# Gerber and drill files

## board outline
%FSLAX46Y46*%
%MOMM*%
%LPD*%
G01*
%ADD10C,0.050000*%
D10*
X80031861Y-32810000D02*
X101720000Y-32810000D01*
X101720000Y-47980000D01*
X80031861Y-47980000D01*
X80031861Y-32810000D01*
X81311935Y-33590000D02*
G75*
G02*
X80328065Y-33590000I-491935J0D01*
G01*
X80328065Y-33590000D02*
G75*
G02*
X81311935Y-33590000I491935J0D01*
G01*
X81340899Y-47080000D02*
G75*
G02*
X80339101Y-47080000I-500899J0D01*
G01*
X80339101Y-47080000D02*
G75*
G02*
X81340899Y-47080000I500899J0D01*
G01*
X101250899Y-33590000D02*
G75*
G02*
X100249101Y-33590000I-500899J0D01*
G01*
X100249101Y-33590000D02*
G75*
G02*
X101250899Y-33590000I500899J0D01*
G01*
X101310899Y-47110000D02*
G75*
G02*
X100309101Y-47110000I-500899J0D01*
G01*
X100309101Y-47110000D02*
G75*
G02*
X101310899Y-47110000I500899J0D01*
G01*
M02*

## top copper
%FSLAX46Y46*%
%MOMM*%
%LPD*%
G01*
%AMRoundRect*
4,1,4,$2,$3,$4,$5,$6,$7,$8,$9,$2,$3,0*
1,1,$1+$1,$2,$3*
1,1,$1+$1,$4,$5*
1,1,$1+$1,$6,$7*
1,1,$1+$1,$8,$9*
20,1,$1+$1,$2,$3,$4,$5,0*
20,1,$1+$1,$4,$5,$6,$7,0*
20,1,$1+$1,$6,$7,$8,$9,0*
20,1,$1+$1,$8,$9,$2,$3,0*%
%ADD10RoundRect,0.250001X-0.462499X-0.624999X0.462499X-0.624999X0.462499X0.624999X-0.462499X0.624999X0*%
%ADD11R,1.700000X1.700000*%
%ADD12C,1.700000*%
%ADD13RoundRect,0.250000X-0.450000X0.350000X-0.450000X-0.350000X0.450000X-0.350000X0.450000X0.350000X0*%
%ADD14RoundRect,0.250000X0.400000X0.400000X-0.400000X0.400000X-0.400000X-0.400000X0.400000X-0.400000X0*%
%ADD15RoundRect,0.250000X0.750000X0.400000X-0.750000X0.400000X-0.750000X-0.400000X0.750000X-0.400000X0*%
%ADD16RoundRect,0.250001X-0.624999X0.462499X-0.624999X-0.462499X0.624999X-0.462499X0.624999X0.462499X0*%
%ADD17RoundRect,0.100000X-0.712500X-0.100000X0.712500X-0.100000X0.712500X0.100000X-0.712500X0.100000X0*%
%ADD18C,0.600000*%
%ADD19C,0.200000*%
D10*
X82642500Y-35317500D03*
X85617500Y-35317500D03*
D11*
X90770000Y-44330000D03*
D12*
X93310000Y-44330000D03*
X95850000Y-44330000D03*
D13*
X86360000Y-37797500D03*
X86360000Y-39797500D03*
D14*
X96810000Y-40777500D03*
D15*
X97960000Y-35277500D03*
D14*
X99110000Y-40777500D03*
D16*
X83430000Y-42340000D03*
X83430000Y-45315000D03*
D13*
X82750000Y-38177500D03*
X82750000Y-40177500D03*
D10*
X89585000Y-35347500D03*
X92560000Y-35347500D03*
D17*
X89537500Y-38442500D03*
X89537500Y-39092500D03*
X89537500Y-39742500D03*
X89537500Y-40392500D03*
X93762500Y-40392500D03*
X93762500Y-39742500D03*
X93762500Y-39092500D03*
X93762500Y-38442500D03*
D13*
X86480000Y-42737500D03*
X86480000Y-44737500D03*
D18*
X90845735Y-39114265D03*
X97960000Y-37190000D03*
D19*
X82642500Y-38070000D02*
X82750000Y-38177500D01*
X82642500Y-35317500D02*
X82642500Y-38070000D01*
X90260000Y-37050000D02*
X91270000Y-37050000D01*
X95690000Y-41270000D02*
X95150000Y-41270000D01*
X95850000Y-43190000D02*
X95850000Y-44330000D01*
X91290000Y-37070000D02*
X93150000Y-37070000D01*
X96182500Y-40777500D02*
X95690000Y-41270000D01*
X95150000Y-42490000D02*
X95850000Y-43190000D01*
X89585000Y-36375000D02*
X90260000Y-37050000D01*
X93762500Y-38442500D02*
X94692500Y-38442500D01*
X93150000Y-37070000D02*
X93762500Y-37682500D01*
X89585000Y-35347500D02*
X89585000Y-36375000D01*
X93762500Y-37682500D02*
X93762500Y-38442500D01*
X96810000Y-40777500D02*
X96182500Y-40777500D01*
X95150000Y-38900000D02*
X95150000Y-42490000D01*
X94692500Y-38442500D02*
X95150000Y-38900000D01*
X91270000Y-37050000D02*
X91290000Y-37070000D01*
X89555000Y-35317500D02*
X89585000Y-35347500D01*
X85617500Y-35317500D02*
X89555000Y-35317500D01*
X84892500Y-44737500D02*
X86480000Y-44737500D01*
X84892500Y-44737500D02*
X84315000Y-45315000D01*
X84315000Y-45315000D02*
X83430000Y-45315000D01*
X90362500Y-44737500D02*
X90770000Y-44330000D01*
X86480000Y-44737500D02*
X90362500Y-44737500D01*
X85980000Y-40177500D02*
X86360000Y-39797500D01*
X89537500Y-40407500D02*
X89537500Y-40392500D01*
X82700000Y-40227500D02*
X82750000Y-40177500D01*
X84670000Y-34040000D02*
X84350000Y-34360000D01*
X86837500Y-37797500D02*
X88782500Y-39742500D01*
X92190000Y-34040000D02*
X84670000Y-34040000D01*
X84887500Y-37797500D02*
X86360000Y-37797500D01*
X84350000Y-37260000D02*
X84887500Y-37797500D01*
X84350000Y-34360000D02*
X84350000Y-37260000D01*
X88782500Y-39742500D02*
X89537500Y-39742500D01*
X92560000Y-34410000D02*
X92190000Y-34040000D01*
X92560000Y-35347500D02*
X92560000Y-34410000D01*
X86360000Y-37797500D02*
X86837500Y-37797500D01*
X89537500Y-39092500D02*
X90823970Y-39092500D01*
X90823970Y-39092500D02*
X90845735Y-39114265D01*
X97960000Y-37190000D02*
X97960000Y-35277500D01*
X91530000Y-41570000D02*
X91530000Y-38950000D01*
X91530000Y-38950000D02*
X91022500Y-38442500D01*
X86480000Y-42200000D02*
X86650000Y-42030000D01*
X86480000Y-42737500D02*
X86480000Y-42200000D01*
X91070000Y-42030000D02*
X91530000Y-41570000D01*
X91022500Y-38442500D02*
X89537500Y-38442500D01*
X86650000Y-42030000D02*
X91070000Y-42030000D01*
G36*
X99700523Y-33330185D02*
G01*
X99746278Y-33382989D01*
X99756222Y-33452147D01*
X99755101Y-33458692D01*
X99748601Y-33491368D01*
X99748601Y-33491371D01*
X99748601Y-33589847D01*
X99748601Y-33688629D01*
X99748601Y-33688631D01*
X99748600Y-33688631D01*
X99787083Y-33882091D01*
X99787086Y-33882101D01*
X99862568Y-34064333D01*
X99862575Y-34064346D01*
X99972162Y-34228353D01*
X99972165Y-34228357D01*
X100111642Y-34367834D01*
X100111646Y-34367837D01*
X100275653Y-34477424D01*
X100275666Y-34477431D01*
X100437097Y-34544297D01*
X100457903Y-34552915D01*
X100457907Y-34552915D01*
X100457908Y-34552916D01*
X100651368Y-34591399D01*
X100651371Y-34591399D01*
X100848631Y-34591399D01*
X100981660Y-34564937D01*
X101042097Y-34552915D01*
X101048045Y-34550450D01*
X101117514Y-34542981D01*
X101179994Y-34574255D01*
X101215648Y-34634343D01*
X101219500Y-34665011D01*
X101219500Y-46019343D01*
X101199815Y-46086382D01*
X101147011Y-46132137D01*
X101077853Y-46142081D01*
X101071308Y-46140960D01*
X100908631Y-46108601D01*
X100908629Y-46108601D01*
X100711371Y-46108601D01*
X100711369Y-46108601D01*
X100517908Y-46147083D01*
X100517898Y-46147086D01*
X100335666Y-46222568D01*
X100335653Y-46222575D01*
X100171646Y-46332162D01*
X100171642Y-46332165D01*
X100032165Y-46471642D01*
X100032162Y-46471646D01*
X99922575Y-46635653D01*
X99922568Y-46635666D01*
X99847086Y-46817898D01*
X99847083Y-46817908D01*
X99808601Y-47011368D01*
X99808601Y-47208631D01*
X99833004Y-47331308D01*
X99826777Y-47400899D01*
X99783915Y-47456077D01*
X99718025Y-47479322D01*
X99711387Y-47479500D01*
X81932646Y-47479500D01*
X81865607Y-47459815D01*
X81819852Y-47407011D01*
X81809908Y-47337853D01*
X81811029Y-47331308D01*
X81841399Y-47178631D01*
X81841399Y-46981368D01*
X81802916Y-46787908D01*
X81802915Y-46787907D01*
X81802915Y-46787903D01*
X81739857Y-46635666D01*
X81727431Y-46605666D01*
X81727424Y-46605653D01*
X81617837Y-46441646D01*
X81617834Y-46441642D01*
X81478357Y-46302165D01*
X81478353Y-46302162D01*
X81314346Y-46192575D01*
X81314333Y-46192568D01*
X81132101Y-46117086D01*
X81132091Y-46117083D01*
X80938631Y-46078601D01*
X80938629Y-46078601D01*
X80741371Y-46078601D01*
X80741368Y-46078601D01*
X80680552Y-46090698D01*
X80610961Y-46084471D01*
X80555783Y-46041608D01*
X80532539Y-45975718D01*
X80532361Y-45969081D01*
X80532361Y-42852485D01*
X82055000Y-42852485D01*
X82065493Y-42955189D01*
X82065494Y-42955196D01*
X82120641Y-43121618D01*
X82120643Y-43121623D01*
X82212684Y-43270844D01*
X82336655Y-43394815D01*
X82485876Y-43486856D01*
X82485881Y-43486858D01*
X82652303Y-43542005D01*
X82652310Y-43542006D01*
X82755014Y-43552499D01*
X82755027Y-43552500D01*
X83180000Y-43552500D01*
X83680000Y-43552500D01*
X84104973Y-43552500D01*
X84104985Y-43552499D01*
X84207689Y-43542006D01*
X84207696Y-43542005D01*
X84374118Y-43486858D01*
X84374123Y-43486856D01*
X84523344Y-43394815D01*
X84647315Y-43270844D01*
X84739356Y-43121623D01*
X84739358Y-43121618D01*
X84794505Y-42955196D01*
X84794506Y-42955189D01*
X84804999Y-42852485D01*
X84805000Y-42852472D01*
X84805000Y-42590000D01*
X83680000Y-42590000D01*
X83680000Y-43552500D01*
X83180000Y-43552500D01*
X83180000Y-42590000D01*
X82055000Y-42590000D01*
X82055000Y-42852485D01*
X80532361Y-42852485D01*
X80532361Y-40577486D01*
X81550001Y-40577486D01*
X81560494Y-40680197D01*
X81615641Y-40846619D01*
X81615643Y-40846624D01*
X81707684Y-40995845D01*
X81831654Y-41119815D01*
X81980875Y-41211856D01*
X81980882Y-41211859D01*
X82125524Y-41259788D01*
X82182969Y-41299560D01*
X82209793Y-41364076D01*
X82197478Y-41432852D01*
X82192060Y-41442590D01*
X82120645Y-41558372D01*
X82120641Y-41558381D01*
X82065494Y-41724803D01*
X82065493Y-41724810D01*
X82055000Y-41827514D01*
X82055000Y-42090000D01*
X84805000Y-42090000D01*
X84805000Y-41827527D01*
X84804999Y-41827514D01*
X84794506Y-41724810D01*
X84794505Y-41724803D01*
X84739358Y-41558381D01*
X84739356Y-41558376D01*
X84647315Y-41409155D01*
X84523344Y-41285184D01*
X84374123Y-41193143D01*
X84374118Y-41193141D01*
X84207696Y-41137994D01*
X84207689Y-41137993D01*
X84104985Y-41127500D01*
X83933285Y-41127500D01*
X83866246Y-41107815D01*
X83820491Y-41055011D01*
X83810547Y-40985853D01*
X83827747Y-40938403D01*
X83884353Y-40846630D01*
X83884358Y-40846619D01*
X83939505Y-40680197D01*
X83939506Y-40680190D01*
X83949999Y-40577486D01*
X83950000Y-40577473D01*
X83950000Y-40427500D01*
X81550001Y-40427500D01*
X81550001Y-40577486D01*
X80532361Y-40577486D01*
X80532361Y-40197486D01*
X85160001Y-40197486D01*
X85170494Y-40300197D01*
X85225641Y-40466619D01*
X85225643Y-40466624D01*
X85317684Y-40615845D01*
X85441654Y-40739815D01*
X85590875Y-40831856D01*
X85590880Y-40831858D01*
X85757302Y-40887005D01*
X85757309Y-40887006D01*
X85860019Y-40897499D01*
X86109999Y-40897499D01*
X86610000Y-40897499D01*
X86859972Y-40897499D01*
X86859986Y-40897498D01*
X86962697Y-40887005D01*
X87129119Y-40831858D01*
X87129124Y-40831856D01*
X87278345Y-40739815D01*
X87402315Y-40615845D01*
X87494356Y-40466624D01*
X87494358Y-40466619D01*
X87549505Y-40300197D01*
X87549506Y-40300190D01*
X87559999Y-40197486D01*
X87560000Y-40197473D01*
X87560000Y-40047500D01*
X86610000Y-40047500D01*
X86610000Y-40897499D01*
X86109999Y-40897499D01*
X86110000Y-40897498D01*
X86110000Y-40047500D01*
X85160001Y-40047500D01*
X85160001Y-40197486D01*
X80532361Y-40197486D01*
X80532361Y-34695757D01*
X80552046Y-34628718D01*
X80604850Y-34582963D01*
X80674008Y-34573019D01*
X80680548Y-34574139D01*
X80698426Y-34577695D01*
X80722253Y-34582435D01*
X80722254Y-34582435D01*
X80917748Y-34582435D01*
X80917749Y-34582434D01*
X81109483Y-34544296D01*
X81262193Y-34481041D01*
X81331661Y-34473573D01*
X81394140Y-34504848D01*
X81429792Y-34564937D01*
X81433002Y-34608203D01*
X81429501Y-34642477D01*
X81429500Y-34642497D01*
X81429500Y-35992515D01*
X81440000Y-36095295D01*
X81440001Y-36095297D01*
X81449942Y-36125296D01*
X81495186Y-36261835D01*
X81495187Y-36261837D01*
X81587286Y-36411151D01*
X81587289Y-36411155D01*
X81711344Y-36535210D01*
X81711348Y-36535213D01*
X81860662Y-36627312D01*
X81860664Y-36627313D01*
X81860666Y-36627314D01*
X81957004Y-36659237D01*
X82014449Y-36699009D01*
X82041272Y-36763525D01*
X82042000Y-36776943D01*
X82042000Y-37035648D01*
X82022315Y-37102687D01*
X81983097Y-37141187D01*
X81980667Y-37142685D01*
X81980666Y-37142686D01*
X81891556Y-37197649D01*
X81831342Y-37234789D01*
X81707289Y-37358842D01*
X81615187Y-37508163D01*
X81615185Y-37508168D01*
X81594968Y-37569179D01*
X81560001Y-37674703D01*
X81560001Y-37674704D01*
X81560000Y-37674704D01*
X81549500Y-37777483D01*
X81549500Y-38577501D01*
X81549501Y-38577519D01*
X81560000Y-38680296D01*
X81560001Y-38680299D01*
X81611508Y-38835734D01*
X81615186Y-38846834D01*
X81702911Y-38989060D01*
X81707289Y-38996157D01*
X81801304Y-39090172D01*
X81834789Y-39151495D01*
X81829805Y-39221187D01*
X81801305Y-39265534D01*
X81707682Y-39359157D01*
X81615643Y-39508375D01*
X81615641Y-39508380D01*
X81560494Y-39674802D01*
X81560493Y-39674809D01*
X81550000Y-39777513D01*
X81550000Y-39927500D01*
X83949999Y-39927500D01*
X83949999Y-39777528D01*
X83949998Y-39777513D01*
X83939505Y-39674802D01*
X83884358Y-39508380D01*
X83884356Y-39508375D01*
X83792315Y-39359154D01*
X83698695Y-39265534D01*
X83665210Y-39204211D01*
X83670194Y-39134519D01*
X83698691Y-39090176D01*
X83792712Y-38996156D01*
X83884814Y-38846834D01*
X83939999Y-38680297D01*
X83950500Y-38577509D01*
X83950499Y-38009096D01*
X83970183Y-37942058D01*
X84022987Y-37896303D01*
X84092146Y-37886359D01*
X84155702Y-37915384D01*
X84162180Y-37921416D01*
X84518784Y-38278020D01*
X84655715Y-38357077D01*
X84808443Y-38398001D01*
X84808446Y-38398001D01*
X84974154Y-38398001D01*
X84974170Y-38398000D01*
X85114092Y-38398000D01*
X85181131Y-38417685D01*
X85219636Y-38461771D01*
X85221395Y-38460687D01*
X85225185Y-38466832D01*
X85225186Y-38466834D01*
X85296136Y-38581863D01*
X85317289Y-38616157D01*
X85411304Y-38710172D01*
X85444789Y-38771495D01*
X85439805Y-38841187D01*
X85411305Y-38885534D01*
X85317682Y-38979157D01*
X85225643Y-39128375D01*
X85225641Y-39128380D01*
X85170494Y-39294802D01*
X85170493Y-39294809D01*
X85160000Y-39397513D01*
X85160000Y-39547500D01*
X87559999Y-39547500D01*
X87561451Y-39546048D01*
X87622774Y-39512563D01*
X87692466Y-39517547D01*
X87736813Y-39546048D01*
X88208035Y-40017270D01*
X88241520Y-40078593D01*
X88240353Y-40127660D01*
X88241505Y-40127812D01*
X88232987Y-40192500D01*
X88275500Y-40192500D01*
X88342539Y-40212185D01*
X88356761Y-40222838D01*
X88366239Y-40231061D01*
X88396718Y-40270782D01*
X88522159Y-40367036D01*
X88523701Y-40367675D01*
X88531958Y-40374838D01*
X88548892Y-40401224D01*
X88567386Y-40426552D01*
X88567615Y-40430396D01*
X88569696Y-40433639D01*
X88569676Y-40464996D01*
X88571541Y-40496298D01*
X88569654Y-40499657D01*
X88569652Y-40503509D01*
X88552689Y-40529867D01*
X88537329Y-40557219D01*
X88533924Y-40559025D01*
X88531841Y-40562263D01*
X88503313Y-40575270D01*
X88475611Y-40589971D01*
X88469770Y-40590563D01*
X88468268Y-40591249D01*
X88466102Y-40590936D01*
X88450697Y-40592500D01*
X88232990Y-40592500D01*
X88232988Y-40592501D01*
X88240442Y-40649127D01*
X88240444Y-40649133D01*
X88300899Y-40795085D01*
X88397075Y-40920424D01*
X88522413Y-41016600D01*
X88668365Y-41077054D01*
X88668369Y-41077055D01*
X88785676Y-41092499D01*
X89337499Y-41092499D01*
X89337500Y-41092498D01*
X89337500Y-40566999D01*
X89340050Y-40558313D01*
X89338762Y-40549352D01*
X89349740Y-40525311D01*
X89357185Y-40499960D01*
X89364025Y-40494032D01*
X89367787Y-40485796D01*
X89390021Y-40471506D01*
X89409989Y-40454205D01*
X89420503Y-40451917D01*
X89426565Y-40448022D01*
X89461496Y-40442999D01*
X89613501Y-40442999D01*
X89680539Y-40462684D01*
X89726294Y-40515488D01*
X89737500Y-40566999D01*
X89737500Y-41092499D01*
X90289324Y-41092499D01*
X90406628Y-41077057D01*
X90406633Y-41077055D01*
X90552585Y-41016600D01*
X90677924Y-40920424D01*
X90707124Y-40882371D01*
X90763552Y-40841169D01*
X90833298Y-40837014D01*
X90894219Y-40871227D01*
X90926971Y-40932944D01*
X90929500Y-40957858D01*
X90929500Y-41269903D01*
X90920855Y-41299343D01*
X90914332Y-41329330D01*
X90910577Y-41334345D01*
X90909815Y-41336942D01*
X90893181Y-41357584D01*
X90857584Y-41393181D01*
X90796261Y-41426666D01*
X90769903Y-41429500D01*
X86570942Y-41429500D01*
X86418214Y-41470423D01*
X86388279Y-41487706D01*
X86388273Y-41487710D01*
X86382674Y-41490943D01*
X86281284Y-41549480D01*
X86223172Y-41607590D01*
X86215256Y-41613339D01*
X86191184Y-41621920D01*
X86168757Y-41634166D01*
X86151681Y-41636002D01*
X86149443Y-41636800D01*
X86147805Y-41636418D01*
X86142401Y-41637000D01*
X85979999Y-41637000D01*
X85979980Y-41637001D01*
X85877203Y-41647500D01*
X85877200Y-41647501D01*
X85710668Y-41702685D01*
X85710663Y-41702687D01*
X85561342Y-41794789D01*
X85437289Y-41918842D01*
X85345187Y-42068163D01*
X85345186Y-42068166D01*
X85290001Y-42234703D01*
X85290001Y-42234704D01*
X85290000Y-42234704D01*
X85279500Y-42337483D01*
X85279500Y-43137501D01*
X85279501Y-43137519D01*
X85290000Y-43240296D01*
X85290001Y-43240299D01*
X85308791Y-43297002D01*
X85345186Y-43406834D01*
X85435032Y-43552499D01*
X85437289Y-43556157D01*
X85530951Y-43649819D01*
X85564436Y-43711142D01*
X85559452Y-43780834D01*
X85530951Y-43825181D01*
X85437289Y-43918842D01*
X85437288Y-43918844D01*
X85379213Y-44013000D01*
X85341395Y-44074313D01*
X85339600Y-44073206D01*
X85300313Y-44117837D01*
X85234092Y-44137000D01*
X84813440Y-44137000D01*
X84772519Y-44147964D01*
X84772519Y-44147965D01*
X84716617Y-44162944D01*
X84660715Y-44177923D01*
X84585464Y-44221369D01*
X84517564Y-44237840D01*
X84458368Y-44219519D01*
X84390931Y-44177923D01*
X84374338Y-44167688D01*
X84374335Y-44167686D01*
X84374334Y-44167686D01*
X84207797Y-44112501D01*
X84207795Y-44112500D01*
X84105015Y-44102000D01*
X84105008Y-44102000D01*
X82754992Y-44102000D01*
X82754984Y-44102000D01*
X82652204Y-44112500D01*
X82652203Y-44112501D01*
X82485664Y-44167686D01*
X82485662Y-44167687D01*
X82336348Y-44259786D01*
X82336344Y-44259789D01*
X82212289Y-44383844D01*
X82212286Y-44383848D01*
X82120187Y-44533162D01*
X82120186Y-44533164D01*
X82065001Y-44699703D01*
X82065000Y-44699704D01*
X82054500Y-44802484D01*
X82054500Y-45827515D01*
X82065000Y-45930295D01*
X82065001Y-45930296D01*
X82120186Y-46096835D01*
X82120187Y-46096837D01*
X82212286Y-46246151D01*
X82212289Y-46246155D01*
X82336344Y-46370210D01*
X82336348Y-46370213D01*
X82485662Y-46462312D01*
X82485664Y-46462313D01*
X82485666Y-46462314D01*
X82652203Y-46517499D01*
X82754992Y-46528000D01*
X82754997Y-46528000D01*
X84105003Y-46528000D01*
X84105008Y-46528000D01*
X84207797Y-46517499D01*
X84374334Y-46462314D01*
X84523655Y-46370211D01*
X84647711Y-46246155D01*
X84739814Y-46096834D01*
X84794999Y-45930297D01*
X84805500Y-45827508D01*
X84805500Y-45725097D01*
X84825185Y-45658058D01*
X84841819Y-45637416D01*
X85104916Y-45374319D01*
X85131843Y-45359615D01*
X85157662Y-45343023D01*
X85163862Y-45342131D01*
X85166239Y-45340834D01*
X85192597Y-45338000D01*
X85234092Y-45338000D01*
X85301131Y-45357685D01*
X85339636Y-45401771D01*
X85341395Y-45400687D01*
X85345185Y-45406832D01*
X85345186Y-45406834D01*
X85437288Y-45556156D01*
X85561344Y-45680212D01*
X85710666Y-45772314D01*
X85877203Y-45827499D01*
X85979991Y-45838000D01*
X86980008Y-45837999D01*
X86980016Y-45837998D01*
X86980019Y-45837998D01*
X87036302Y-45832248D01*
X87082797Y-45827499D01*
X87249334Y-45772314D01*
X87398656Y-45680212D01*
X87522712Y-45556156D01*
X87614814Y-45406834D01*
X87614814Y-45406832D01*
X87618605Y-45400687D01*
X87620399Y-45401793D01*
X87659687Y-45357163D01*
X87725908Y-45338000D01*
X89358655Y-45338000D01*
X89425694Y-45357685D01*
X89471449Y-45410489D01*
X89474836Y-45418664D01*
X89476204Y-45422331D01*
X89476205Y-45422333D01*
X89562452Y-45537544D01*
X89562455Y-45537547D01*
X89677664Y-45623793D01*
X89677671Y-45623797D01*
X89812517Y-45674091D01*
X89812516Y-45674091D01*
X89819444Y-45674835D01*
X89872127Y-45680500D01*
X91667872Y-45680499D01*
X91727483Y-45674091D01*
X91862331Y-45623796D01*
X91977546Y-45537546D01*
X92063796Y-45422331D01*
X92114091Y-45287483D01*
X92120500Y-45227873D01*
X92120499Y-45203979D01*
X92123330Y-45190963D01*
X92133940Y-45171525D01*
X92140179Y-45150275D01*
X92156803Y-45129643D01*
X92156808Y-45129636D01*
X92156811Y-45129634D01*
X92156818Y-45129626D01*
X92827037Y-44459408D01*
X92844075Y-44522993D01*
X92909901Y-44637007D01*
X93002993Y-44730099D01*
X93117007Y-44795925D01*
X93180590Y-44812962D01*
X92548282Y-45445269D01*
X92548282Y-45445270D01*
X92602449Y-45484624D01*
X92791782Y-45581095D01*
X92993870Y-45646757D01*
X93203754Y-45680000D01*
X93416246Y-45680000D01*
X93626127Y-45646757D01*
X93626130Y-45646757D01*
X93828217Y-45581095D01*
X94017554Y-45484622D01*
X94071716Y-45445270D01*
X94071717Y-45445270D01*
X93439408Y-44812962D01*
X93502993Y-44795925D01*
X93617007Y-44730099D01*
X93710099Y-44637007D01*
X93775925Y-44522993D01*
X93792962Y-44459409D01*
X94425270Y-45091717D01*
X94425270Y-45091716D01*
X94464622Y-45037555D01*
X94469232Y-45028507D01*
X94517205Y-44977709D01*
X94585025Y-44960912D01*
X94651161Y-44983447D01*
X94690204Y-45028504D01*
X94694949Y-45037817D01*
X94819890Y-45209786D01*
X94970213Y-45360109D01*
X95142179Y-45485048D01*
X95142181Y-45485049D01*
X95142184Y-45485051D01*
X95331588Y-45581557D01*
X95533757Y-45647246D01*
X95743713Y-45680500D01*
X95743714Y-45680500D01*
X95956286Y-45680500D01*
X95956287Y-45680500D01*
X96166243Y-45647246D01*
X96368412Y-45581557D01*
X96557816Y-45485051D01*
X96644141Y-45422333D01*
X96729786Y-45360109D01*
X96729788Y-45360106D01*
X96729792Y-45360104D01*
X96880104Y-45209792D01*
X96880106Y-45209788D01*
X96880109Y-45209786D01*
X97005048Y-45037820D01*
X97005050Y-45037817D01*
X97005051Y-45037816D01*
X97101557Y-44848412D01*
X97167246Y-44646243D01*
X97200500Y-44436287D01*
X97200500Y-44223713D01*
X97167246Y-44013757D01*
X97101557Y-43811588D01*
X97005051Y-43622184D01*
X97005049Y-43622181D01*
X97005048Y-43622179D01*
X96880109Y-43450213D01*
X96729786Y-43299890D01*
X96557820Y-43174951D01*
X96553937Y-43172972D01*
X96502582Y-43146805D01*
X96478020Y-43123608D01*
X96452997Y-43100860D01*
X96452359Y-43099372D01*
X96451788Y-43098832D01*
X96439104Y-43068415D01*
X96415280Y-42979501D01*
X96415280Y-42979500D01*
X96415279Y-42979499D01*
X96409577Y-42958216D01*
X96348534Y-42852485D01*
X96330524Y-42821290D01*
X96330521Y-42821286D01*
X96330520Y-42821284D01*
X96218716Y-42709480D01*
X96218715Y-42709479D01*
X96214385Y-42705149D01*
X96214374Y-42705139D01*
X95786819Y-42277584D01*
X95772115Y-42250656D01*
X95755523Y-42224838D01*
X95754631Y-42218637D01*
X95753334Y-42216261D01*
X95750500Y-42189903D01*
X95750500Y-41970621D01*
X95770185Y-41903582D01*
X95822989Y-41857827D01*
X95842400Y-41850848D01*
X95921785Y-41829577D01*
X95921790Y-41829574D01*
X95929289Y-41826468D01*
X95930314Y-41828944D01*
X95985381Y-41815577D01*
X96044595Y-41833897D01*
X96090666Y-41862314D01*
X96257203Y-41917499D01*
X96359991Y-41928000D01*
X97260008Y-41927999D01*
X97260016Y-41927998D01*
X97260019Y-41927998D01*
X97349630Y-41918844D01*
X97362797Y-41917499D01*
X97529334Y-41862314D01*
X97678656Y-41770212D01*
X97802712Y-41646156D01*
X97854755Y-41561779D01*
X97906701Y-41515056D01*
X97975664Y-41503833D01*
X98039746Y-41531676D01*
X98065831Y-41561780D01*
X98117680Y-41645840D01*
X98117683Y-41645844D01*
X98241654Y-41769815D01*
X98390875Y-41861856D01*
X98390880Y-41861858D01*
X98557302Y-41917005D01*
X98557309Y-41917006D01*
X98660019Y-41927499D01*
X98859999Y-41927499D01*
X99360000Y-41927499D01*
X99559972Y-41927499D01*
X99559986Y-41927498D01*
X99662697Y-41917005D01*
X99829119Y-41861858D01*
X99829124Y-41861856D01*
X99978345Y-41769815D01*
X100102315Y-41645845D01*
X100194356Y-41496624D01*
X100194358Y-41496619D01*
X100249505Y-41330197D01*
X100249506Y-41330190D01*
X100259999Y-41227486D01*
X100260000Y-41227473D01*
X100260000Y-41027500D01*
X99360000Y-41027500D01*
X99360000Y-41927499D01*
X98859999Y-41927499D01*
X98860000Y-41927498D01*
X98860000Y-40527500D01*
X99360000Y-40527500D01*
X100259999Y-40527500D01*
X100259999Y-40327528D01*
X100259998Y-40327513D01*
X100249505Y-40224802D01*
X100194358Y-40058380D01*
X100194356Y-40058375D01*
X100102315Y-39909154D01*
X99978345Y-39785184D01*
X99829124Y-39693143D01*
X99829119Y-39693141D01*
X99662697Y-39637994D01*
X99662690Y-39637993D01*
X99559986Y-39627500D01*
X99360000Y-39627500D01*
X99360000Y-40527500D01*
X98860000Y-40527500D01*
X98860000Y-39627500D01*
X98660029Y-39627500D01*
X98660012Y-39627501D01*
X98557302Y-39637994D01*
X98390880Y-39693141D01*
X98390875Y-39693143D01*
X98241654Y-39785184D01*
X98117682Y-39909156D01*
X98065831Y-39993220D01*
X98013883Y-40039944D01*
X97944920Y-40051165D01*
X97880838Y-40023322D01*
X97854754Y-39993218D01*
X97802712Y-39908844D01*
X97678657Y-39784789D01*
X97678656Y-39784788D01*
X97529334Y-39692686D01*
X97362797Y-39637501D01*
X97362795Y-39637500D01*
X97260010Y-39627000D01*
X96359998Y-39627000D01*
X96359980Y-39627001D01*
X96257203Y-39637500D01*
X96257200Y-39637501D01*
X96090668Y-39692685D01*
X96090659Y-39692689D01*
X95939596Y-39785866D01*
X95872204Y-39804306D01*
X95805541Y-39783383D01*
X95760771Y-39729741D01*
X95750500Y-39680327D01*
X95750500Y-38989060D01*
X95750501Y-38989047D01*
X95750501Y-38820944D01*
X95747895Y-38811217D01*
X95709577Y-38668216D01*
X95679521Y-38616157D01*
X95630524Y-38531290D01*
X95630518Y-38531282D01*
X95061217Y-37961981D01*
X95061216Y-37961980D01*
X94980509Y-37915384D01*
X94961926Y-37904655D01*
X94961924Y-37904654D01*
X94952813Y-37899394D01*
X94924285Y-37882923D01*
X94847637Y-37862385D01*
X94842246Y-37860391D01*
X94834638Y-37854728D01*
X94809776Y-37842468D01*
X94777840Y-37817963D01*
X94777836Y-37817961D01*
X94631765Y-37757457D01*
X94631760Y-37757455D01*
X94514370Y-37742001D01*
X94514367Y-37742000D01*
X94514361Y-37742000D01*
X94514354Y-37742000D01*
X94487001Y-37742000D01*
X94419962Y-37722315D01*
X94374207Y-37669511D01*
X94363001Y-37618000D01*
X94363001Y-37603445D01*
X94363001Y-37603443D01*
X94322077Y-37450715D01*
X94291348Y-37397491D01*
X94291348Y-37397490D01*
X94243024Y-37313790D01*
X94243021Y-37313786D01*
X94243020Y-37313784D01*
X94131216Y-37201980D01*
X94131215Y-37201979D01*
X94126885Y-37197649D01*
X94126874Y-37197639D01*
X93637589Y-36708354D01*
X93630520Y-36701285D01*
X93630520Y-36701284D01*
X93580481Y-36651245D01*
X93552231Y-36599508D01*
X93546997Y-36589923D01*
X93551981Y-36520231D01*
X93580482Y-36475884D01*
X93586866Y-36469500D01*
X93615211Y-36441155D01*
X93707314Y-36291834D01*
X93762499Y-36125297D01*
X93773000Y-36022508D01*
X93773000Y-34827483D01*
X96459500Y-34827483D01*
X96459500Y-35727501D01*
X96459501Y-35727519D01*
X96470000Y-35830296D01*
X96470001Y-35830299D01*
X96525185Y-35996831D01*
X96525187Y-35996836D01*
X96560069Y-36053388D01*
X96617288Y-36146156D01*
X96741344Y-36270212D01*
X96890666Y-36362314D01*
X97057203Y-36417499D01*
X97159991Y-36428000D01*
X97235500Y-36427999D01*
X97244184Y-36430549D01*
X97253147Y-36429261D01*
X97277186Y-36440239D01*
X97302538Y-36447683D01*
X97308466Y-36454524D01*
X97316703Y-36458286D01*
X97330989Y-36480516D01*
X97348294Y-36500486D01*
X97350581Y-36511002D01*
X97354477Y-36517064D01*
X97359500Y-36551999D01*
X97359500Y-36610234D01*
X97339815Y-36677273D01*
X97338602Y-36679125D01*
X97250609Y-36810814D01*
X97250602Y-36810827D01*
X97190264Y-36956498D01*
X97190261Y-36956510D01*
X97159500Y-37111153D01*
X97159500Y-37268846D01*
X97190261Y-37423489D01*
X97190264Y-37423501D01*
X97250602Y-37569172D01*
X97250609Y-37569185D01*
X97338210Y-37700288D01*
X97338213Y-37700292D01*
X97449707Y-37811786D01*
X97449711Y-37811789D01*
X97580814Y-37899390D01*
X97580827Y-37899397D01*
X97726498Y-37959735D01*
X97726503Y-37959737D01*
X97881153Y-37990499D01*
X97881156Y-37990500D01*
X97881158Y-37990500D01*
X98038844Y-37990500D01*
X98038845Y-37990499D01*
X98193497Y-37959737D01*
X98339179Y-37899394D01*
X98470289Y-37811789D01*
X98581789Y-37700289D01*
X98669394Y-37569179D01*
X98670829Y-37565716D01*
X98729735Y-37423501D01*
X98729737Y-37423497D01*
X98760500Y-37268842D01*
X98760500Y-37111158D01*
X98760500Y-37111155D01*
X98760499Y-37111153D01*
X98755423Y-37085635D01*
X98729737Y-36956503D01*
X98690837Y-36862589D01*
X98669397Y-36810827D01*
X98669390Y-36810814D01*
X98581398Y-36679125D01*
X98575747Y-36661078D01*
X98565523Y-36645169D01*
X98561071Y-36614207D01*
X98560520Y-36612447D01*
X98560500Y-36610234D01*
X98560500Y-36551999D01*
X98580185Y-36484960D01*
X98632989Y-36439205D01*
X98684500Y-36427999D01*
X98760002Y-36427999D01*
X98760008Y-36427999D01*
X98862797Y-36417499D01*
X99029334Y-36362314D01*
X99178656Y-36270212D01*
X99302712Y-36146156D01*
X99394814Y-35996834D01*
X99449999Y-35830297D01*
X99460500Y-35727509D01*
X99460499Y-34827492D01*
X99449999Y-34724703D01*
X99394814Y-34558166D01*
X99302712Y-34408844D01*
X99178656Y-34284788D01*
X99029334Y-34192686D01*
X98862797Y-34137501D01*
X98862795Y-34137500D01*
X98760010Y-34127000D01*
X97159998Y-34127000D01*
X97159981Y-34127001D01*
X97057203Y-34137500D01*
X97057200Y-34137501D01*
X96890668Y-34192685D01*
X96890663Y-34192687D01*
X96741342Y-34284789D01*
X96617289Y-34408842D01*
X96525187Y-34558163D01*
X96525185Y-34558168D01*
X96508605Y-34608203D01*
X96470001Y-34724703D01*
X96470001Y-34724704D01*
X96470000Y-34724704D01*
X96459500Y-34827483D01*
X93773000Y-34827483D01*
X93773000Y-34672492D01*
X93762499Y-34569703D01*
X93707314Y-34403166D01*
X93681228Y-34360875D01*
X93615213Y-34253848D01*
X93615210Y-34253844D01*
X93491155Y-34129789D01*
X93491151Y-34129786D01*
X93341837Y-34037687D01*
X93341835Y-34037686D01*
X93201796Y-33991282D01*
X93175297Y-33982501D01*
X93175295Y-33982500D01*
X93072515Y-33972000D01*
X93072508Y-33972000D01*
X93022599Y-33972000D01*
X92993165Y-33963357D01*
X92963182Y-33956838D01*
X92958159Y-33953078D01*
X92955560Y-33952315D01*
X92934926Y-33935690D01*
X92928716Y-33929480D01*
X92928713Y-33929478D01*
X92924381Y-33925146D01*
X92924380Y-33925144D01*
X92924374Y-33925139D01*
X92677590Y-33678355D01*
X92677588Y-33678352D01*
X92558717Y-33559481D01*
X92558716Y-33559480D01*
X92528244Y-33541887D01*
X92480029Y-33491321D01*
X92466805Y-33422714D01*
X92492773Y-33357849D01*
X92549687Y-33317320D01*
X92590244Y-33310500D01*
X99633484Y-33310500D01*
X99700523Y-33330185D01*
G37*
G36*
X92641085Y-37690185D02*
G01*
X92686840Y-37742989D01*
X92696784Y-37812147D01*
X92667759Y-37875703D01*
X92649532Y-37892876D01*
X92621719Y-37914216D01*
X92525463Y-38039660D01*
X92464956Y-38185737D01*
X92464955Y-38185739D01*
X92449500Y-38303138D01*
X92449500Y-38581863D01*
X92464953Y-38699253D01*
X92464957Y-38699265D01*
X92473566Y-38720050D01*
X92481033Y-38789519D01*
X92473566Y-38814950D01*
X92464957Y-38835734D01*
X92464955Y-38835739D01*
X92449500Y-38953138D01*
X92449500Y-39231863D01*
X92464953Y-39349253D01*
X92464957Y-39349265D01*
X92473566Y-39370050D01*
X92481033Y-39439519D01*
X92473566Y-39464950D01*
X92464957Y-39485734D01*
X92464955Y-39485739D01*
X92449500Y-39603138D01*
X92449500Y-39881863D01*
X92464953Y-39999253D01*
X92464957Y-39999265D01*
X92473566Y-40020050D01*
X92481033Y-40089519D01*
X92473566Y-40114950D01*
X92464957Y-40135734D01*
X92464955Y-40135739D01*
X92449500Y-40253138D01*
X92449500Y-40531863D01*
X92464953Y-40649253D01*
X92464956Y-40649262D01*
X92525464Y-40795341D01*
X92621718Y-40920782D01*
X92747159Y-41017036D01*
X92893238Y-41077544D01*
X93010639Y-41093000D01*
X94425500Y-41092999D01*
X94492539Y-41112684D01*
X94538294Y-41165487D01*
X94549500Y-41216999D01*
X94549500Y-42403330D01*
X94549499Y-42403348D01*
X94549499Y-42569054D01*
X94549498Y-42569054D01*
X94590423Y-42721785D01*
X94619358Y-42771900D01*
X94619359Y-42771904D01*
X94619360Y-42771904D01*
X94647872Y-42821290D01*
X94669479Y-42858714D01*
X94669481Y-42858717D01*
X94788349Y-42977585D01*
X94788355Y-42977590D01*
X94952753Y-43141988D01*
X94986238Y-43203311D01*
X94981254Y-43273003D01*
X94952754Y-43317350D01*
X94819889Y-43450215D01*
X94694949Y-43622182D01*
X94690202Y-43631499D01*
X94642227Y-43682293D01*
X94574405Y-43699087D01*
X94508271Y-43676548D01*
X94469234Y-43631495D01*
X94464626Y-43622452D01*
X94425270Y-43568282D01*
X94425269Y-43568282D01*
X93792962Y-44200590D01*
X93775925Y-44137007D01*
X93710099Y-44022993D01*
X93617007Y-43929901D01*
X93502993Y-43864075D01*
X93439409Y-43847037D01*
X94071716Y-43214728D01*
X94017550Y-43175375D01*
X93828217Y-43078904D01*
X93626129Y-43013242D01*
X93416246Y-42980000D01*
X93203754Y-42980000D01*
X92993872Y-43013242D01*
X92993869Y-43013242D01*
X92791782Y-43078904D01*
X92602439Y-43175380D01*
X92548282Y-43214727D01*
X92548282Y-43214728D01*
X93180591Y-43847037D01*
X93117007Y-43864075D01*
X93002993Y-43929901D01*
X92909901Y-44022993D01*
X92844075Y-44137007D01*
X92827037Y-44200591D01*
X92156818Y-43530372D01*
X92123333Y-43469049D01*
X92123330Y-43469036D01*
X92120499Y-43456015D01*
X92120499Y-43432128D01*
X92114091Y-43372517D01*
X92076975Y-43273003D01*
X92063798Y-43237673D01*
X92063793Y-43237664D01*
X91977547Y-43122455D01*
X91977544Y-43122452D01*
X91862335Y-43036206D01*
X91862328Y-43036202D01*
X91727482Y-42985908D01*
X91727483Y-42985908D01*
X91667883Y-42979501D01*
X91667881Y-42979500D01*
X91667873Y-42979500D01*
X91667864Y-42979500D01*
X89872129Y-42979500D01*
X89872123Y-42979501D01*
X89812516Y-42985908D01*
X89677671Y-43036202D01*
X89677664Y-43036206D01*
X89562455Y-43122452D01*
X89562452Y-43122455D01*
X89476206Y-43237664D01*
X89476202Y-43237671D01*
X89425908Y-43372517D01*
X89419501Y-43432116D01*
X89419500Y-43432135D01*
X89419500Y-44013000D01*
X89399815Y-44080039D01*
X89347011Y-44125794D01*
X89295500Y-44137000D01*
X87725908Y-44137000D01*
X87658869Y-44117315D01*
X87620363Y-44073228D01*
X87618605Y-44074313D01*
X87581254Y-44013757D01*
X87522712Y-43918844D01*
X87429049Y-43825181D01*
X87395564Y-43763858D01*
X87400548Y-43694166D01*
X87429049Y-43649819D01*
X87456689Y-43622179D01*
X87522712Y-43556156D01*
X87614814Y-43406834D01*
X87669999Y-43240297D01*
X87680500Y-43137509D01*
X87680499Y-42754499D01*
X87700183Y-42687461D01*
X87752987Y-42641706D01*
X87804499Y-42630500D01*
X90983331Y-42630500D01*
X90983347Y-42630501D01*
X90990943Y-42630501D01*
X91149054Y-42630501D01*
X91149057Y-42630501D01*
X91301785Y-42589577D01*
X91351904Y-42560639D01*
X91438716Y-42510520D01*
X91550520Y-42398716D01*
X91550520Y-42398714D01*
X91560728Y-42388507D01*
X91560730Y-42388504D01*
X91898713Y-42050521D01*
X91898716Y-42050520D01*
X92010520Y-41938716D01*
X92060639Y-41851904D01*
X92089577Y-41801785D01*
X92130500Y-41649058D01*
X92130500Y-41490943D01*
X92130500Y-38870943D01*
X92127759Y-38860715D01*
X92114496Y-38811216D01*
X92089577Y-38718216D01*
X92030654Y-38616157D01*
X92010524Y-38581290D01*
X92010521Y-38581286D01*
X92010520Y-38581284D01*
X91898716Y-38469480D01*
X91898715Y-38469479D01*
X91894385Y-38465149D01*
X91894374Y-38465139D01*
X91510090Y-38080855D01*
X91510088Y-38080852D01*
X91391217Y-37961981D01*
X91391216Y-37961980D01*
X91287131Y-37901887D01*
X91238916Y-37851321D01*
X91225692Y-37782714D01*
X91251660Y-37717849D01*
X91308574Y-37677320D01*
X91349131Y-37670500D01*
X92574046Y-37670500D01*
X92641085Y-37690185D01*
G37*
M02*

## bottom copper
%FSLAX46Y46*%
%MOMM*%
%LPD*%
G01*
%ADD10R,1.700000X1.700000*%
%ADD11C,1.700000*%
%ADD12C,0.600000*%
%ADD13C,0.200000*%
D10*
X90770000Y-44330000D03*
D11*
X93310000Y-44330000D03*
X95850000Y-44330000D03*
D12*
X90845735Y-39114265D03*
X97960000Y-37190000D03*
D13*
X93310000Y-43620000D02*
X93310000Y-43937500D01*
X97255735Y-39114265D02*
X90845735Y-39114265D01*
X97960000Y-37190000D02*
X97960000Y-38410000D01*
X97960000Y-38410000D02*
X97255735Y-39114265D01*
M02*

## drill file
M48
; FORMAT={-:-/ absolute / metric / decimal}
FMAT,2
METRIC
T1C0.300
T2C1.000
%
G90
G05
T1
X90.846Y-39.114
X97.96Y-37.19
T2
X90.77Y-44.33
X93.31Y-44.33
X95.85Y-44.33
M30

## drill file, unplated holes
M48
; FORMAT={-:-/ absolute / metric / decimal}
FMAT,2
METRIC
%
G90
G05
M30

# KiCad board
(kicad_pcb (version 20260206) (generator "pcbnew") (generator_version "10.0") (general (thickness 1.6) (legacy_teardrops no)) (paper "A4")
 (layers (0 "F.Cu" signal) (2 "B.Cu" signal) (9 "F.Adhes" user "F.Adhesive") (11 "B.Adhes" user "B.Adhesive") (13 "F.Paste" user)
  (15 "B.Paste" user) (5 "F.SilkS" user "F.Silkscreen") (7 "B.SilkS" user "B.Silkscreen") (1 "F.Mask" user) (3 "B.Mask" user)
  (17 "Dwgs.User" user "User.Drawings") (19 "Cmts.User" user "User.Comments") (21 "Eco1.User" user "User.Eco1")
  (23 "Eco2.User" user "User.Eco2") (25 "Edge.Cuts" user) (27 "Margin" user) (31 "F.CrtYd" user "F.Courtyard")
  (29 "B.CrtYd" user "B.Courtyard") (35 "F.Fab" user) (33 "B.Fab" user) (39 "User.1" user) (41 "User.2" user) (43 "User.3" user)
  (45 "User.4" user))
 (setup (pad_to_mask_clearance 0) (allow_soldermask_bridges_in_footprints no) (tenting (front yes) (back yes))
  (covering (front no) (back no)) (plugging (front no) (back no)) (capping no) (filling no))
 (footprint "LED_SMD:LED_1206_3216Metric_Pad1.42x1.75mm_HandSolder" (layer "F.Cu") (at 84.13 35.3175)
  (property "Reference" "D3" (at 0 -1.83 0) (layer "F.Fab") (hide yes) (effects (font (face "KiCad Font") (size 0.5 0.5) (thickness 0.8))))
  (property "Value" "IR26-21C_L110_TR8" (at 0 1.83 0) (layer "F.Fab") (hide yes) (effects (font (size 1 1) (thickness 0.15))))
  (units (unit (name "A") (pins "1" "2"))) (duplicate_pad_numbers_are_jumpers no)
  (pad "1" smd roundrect (at -1.4875 0) (size 1.425 1.75) (layers "F.Cu" "F.Mask" "F.Paste") (roundrect_rratio 0.175439) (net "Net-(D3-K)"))
  (pad "2" smd roundrect (at 1.4875 0) (size 1.425 1.75) (layers "F.Cu" "F.Mask" "F.Paste") (roundrect_rratio 0.175439) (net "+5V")))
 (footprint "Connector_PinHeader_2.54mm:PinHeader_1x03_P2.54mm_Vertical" (layer "F.Cu") (at 90.77 44.33 90)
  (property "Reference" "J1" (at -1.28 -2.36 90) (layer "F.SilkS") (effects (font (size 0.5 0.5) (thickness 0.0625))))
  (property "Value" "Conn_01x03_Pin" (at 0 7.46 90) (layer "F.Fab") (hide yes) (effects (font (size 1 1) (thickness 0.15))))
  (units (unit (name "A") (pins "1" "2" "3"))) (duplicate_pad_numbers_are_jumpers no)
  (pad "1" thru_hole rect (at 0 0 90) (size 1.7 1.7) (drill 1) (layers "*.Cu" "*.Mask") (remove_unused_layers no) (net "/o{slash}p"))
  (pad "2" thru_hole circle (at 0 2.54 90) (size 1.7 1.7) (drill 1) (layers "*.Cu" "*.Mask") (remove_unused_layers no) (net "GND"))
  (pad "3" thru_hole circle (at 0 5.08 90) (size 1.7 1.7) (drill 1) (layers "*.Cu" "*.Mask") (remove_unused_layers no) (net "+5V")))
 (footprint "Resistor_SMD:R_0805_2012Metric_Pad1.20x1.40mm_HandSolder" (layer "F.Cu") (at 86.36 38.7975 -90)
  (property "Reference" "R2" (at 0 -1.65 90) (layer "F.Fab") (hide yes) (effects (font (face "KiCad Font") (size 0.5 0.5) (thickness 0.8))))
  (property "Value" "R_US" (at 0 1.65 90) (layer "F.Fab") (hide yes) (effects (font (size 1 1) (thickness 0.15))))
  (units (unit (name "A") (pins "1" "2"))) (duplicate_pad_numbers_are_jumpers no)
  (pad "1" smd roundrect (at -1 0 270) (size 1.2 1.4) (layers "F.Cu" "F.Mask" "F.Paste") (roundrect_rratio 0.208333) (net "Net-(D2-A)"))
  (pad "2" smd roundrect (at 1 0 270) (size 1.2 1.4) (layers "F.Cu" "F.Mask" "F.Paste") (roundrect_rratio 0.208333) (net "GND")))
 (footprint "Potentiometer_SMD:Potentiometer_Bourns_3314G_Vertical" (layer "F.Cu") (at 97.96 38.0275 180)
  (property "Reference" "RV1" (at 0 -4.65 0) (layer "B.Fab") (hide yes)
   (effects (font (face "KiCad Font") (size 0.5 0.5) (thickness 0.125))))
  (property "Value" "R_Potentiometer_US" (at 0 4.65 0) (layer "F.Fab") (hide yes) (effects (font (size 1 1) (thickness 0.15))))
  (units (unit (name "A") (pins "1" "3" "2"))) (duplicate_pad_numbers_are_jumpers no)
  (pad "1" smd roundrect (at 1.15 -2.75 180) (size 1.3 1.3) (layers "F.Cu" "F.Mask" "F.Paste") (roundrect_rratio 0.192308) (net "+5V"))
  (pad "2" smd roundrect (at 0 2.75 180) (size 2 1.3) (layers "F.Cu" "F.Mask" "F.Paste") (roundrect_rratio 0.192308) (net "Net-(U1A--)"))
  (pad "3" smd roundrect (at -1.15 -2.75 180) (size 1.3 1.3) (layers "F.Cu" "F.Mask" "F.Paste") (roundrect_rratio 0.192308) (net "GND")))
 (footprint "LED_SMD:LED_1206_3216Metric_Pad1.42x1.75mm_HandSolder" (layer "F.Cu") (at 83.43 43.8275 -90)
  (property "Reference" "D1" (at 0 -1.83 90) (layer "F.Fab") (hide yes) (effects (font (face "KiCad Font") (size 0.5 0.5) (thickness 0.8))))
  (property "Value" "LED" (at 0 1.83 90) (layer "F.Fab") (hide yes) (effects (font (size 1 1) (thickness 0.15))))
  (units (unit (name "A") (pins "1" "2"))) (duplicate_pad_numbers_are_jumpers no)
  (pad "1" smd roundrect (at -1.4875 0 270) (size 1.425 1.75) (layers "F.Cu" "F.Mask" "F.Paste") (roundrect_rratio 0.175439) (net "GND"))
  (pad "2" smd roundrect (at 1.4875 0 270) (size 1.425 1.75) (layers "F.Cu" "F.Mask" "F.Paste") (roundrect_rratio 0.175439)
   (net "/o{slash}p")))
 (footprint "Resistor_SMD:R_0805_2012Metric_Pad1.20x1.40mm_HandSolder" (layer "F.Cu") (at 82.75 39.1775 -90)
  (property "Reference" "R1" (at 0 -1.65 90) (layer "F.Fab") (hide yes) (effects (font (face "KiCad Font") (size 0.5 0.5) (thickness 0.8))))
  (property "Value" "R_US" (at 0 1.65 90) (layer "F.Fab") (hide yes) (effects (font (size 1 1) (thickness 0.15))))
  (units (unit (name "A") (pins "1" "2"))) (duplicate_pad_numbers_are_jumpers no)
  (pad "1" smd roundrect (at -1 0 270) (size 1.2 1.4) (layers "F.Cu" "F.Mask" "F.Paste") (roundrect_rratio 0.208333) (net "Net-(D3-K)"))
  (pad "2" smd roundrect (at 1 0 270) (size 1.2 1.4) (layers "F.Cu" "F.Mask" "F.Paste") (roundrect_rratio 0.208333) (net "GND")))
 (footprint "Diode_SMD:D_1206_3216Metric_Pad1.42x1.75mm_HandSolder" (layer "F.Cu") (at 91.0725 35.3475)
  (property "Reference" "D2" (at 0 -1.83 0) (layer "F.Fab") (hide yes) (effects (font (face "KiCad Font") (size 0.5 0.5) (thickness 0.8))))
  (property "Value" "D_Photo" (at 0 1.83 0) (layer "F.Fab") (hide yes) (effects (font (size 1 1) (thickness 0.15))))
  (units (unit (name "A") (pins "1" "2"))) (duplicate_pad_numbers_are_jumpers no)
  (pad "1" smd roundrect (at -1.4875 0) (size 1.425 1.75) (layers "F.Cu" "F.Mask" "F.Paste") (roundrect_rratio 0.175439) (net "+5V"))
  (pad "2" smd roundrect (at 1.4875 0) (size 1.425 1.75) (layers "F.Cu" "F.Mask" "F.Paste") (roundrect_rratio 0.175439) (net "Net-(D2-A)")))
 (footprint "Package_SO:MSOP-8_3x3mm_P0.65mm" (layer "F.Cu") (at 91.65 39.4175)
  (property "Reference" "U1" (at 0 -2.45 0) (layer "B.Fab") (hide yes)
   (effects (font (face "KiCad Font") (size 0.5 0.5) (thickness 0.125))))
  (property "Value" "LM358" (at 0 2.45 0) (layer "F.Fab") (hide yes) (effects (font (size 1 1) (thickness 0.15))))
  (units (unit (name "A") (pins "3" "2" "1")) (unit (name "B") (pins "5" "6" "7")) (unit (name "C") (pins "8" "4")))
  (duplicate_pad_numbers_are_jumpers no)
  (pad "1" smd roundrect (at -2.1125 -0.975) (size 1.625 0.4) (layers "F.Cu" "F.Mask" "F.Paste") (roundrect_rratio 0.25)
   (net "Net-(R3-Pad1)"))
  (pad "2" smd roundrect (at -2.1125 -0.325) (size 1.625 0.4) (layers "F.Cu" "F.Mask" "F.Paste") (roundrect_rratio 0.25) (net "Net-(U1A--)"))
  (pad "3" smd roundrect (at -2.1125 0.325) (size 1.625 0.4) (layers "F.Cu" "F.Mask" "F.Paste") (roundrect_rratio 0.25) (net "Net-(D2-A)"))
  (pad "4" smd roundrect (at -2.1125 0.975) (size 1.625 0.4) (layers "F.Cu" "F.Mask" "F.Paste") (roundrect_rratio 0.25) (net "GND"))
  (pad "5" smd roundrect (at 2.1125 0.975) (size 1.625 0.4) (layers "F.Cu" "F.Mask" "F.Paste") (roundrect_rratio 0.25))
  (pad "6" smd roundrect (at 2.1125 0.325) (size 1.625 0.4) (layers "F.Cu" "F.Mask" "F.Paste") (roundrect_rratio 0.25))
  (pad "7" smd roundrect (at 2.1125 -0.325) (size 1.625 0.4) (layers "F.Cu" "F.Mask" "F.Paste") (roundrect_rratio 0.25))
  (pad "8" smd roundrect (at 2.1125 -0.975) (size 1.625 0.4) (layers "F.Cu" "F.Mask" "F.Paste") (roundrect_rratio 0.25) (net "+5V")))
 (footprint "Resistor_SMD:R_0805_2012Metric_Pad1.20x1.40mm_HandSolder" (layer "F.Cu") (at 86.48 43.7375 -90)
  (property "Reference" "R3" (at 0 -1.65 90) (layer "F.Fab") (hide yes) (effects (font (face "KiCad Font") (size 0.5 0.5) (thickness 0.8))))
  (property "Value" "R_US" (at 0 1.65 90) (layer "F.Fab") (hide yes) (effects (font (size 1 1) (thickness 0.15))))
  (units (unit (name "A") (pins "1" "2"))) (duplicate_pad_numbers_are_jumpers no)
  (pad "1" smd roundrect (at -1 0 270) (size 1.2 1.4) (layers "F.Cu" "F.Mask" "F.Paste") (roundrect_rratio 0.208333) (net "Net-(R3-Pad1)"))
  (pad "2" smd roundrect (at 1 0 270) (size 1.2 1.4) (layers "F.Cu" "F.Mask" "F.Paste") (roundrect_rratio 0.208333) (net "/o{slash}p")))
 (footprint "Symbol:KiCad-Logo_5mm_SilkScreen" (layer "B.Cu") (at 88.76 36.99 180)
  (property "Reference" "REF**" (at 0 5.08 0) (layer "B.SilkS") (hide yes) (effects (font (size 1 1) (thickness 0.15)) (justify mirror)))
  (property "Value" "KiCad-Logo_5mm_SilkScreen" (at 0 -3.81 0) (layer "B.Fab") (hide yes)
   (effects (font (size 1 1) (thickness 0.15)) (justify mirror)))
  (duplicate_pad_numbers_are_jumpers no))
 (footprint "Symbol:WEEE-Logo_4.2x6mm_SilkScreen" (layer "B.Cu") (at 99.19 42.52 180)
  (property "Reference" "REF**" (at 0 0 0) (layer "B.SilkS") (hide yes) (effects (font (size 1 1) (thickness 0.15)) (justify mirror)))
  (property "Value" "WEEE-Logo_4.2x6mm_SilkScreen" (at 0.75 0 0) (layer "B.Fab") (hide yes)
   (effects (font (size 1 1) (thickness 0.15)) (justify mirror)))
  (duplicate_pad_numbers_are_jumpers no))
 (gr_rect (start 80.031861 32.81) (end 101.72 47.98) (stroke (width 0.05) (type default)) (fill no) (layer "Edge.Cuts"))
 (gr_circle (center 80.82 33.59) (end 81.04 33.15) (stroke (width 0.05) (type default)) (fill no) (layer "Edge.Cuts"))
 (gr_circle (center 80.84 47.08) (end 81.06 47.53) (stroke (width 0.05) (type default)) (fill no) (layer "Edge.Cuts"))
 (gr_circle (center 100.75 33.59) (end 100.97 34.04) (stroke (width 0.05) (type solid)) (fill no) (layer "Edge.Cuts"))
 (gr_circle (center 100.81 47.11) (end 101.03 47.56) (stroke (width 0.05) (type default)) (fill no) (layer "Edge.Cuts"))
 (segment (start 82.6425 38.07) (end 82.75 38.1775) (width 0.2) (layer "F.Cu") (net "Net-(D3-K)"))
 (segment (start 82.6425 35.3175) (end 82.6425 38.07) (width 0.2) (layer "F.Cu") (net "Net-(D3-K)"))
 (segment (start 90.26 37.05) (end 91.27 37.05) (width 0.2) (layer "F.Cu") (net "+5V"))
 (segment (start 95.69 41.27) (end 95.15 41.27) (width 0.2) (layer "F.Cu") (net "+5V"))
 (segment (start 95.85 43.19) (end 95.85 44.33) (width 0.2) (layer "F.Cu") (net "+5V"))
 (segment (start 91.29 37.07) (end 93.15 37.07) (width 0.2) (layer "F.Cu") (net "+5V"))
 (segment (start 96.1825 40.7775) (end 95.69 41.27) (width 0.2) (layer "F.Cu") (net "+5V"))
 (segment (start 95.15 42.49) (end 95.85 43.19) (width 0.2) (layer "F.Cu") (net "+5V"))
 (segment (start 89.585 36.375) (end 90.26 37.05) (width 0.2) (layer "F.Cu") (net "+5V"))
 (segment (start 93.7625 38.4425) (end 94.6925 38.4425) (width 0.2) (layer "F.Cu") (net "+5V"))
 (segment (start 93.15 37.07) (end 93.7625 37.6825) (width 0.2) (layer "F.Cu") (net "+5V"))
 (segment (start 89.585 35.3475) (end 89.585 36.375) (width 0.2) (layer "F.Cu") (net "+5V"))
 (segment (start 93.7625 37.6825) (end 93.7625 38.4425) (width 0.2) (layer "F.Cu") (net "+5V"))
 (segment (start 96.81 40.7775) (end 96.1825 40.7775) (width 0.2) (layer "F.Cu") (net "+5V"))
 (segment (start 95.15 38.9) (end 95.15 42.49) (width 0.2) (layer "F.Cu") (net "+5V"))
 (segment (start 94.6925 38.4425) (end 95.15 38.9) (width 0.2) (layer "F.Cu") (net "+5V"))
 (segment (start 91.27 37.05) (end 91.29 37.07) (width 0.2) (layer "F.Cu") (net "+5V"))
 (segment (start 89.555 35.3175) (end 89.585 35.3475) (width 0.2) (layer "F.Cu") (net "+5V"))
 (segment (start 85.6175 35.3175) (end 89.555 35.3175) (width 0.2) (layer "F.Cu") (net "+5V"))
 (segment (start 84.8925 44.7375) (end 86.48 44.7375) (width 0.2) (layer "F.Cu") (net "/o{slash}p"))
 (segment (start 84.8925 44.7375) (end 84.315 45.315) (width 0.2) (layer "F.Cu") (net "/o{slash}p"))
 (segment (start 84.315 45.315) (end 83.43 45.315) (width 0.2) (layer "F.Cu") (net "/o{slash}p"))
 (segment (start 90.3625 44.7375) (end 90.77 44.33) (width 0.2) (layer "F.Cu") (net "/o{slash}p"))
 (segment (start 86.48 44.7375) (end 90.3625 44.7375) (width 0.2) (layer "F.Cu") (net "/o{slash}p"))
 (segment (start 85.98 40.1775) (end 86.36 39.7975) (width 0.2) (layer "F.Cu") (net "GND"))
 (segment (start 89.5375 40.4075) (end 89.5375 40.3925) (width 0.2) (layer "F.Cu") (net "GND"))
 (segment (start 82.7 40.2275) (end 82.75 40.1775) (width 0.2) (layer "F.Cu") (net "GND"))
 (segment (start 93.31 43.62) (end 93.31 43.9375) (width 0.2) (layer "B.Cu") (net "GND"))
 (segment (start 84.67 34.04) (end 84.35 34.36) (width 0.2) (layer "F.Cu") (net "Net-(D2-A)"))
 (segment (start 86.8375 37.7975) (end 88.7825 39.7425) (width 0.2) (layer "F.Cu") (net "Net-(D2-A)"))
 (segment (start 92.19 34.04) (end 84.67 34.04) (width 0.2) (layer "F.Cu") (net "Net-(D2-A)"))
 (segment (start 84.8875 37.7975) (end 86.36 37.7975) (width 0.2) (layer "F.Cu") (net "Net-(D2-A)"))
 (segment (start 84.35 37.26) (end 84.8875 37.7975) (width 0.2) (layer "F.Cu") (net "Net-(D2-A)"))
 (segment (start 84.35 34.36) (end 84.35 37.26) (width 0.2) (layer "F.Cu") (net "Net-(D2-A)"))
 (segment (start 88.7825 39.7425) (end 89.5375 39.7425) (width 0.2) (layer "F.Cu") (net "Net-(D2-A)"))
 (segment (start 92.56 34.41) (end 92.19 34.04) (width 0.2) (layer "F.Cu") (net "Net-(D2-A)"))
 (segment (start 92.56 35.3475) (end 92.56 34.41) (width 0.2) (layer "F.Cu") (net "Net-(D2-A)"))
 (segment (start 86.36 37.7975) (end 86.8375 37.7975) (width 0.2) (layer "F.Cu") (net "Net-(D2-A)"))
 (segment (start 89.5375 39.0925) (end 90.82397 39.0925) (width 0.2) (layer "F.Cu") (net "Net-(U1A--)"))
 (segment (start 90.82397 39.0925) (end 90.845735 39.114265) (width 0.2) (layer "F.Cu") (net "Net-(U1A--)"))
 (segment (start 97.96 37.19) (end 97.96 35.2775) (width 0.2) (layer "F.Cu") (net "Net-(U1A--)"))
 (via (at 90.845735 39.114265) (size 0.6) (drill 0.3) (layers "F.Cu" "B.Cu") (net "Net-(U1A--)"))
 (via (at 97.96 37.19) (size 0.6) (drill 0.3) (layers "F.Cu" "B.Cu") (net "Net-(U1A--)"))
 (segment (start 97.255735 39.114265) (end 90.845735 39.114265) (width 0.2) (layer "B.Cu") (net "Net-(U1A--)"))
 (segment (start 97.96 37.19) (end 97.96 38.41) (width 0.2) (layer "B.Cu") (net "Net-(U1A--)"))
 (segment (start 97.96 38.41) (end 97.255735 39.114265) (width 0.2) (layer "B.Cu") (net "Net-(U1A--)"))
 (segment (start 91.53 41.57) (end 91.53 38.95) (width 0.2) (layer "F.Cu") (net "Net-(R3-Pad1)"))
 (segment (start 91.53 38.95) (end 91.0225 38.4425) (width 0.2) (layer "F.Cu") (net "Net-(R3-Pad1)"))
 (segment (start 86.48 42.2) (end 86.65 42.03) (width 0.2) (layer "F.Cu") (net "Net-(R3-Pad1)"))
 (segment (start 86.48 42.7375) (end 86.48 42.2) (width 0.2) (layer "F.Cu") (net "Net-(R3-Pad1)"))
 (segment (start 91.07 42.03) (end 91.53 41.57) (width 0.2) (layer "F.Cu") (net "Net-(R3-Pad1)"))
 (segment (start 91.0225 38.4425) (end 89.5375 38.4425) (width 0.2) (layer "F.Cu") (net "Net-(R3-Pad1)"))
 (segment (start 86.65 42.03) (end 91.07 42.03) (width 0.2) (layer "F.Cu") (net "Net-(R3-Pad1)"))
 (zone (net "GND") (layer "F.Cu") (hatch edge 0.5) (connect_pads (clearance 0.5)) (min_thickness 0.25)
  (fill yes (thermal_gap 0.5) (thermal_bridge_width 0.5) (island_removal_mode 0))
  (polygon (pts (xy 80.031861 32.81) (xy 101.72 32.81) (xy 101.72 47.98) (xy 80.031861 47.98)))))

